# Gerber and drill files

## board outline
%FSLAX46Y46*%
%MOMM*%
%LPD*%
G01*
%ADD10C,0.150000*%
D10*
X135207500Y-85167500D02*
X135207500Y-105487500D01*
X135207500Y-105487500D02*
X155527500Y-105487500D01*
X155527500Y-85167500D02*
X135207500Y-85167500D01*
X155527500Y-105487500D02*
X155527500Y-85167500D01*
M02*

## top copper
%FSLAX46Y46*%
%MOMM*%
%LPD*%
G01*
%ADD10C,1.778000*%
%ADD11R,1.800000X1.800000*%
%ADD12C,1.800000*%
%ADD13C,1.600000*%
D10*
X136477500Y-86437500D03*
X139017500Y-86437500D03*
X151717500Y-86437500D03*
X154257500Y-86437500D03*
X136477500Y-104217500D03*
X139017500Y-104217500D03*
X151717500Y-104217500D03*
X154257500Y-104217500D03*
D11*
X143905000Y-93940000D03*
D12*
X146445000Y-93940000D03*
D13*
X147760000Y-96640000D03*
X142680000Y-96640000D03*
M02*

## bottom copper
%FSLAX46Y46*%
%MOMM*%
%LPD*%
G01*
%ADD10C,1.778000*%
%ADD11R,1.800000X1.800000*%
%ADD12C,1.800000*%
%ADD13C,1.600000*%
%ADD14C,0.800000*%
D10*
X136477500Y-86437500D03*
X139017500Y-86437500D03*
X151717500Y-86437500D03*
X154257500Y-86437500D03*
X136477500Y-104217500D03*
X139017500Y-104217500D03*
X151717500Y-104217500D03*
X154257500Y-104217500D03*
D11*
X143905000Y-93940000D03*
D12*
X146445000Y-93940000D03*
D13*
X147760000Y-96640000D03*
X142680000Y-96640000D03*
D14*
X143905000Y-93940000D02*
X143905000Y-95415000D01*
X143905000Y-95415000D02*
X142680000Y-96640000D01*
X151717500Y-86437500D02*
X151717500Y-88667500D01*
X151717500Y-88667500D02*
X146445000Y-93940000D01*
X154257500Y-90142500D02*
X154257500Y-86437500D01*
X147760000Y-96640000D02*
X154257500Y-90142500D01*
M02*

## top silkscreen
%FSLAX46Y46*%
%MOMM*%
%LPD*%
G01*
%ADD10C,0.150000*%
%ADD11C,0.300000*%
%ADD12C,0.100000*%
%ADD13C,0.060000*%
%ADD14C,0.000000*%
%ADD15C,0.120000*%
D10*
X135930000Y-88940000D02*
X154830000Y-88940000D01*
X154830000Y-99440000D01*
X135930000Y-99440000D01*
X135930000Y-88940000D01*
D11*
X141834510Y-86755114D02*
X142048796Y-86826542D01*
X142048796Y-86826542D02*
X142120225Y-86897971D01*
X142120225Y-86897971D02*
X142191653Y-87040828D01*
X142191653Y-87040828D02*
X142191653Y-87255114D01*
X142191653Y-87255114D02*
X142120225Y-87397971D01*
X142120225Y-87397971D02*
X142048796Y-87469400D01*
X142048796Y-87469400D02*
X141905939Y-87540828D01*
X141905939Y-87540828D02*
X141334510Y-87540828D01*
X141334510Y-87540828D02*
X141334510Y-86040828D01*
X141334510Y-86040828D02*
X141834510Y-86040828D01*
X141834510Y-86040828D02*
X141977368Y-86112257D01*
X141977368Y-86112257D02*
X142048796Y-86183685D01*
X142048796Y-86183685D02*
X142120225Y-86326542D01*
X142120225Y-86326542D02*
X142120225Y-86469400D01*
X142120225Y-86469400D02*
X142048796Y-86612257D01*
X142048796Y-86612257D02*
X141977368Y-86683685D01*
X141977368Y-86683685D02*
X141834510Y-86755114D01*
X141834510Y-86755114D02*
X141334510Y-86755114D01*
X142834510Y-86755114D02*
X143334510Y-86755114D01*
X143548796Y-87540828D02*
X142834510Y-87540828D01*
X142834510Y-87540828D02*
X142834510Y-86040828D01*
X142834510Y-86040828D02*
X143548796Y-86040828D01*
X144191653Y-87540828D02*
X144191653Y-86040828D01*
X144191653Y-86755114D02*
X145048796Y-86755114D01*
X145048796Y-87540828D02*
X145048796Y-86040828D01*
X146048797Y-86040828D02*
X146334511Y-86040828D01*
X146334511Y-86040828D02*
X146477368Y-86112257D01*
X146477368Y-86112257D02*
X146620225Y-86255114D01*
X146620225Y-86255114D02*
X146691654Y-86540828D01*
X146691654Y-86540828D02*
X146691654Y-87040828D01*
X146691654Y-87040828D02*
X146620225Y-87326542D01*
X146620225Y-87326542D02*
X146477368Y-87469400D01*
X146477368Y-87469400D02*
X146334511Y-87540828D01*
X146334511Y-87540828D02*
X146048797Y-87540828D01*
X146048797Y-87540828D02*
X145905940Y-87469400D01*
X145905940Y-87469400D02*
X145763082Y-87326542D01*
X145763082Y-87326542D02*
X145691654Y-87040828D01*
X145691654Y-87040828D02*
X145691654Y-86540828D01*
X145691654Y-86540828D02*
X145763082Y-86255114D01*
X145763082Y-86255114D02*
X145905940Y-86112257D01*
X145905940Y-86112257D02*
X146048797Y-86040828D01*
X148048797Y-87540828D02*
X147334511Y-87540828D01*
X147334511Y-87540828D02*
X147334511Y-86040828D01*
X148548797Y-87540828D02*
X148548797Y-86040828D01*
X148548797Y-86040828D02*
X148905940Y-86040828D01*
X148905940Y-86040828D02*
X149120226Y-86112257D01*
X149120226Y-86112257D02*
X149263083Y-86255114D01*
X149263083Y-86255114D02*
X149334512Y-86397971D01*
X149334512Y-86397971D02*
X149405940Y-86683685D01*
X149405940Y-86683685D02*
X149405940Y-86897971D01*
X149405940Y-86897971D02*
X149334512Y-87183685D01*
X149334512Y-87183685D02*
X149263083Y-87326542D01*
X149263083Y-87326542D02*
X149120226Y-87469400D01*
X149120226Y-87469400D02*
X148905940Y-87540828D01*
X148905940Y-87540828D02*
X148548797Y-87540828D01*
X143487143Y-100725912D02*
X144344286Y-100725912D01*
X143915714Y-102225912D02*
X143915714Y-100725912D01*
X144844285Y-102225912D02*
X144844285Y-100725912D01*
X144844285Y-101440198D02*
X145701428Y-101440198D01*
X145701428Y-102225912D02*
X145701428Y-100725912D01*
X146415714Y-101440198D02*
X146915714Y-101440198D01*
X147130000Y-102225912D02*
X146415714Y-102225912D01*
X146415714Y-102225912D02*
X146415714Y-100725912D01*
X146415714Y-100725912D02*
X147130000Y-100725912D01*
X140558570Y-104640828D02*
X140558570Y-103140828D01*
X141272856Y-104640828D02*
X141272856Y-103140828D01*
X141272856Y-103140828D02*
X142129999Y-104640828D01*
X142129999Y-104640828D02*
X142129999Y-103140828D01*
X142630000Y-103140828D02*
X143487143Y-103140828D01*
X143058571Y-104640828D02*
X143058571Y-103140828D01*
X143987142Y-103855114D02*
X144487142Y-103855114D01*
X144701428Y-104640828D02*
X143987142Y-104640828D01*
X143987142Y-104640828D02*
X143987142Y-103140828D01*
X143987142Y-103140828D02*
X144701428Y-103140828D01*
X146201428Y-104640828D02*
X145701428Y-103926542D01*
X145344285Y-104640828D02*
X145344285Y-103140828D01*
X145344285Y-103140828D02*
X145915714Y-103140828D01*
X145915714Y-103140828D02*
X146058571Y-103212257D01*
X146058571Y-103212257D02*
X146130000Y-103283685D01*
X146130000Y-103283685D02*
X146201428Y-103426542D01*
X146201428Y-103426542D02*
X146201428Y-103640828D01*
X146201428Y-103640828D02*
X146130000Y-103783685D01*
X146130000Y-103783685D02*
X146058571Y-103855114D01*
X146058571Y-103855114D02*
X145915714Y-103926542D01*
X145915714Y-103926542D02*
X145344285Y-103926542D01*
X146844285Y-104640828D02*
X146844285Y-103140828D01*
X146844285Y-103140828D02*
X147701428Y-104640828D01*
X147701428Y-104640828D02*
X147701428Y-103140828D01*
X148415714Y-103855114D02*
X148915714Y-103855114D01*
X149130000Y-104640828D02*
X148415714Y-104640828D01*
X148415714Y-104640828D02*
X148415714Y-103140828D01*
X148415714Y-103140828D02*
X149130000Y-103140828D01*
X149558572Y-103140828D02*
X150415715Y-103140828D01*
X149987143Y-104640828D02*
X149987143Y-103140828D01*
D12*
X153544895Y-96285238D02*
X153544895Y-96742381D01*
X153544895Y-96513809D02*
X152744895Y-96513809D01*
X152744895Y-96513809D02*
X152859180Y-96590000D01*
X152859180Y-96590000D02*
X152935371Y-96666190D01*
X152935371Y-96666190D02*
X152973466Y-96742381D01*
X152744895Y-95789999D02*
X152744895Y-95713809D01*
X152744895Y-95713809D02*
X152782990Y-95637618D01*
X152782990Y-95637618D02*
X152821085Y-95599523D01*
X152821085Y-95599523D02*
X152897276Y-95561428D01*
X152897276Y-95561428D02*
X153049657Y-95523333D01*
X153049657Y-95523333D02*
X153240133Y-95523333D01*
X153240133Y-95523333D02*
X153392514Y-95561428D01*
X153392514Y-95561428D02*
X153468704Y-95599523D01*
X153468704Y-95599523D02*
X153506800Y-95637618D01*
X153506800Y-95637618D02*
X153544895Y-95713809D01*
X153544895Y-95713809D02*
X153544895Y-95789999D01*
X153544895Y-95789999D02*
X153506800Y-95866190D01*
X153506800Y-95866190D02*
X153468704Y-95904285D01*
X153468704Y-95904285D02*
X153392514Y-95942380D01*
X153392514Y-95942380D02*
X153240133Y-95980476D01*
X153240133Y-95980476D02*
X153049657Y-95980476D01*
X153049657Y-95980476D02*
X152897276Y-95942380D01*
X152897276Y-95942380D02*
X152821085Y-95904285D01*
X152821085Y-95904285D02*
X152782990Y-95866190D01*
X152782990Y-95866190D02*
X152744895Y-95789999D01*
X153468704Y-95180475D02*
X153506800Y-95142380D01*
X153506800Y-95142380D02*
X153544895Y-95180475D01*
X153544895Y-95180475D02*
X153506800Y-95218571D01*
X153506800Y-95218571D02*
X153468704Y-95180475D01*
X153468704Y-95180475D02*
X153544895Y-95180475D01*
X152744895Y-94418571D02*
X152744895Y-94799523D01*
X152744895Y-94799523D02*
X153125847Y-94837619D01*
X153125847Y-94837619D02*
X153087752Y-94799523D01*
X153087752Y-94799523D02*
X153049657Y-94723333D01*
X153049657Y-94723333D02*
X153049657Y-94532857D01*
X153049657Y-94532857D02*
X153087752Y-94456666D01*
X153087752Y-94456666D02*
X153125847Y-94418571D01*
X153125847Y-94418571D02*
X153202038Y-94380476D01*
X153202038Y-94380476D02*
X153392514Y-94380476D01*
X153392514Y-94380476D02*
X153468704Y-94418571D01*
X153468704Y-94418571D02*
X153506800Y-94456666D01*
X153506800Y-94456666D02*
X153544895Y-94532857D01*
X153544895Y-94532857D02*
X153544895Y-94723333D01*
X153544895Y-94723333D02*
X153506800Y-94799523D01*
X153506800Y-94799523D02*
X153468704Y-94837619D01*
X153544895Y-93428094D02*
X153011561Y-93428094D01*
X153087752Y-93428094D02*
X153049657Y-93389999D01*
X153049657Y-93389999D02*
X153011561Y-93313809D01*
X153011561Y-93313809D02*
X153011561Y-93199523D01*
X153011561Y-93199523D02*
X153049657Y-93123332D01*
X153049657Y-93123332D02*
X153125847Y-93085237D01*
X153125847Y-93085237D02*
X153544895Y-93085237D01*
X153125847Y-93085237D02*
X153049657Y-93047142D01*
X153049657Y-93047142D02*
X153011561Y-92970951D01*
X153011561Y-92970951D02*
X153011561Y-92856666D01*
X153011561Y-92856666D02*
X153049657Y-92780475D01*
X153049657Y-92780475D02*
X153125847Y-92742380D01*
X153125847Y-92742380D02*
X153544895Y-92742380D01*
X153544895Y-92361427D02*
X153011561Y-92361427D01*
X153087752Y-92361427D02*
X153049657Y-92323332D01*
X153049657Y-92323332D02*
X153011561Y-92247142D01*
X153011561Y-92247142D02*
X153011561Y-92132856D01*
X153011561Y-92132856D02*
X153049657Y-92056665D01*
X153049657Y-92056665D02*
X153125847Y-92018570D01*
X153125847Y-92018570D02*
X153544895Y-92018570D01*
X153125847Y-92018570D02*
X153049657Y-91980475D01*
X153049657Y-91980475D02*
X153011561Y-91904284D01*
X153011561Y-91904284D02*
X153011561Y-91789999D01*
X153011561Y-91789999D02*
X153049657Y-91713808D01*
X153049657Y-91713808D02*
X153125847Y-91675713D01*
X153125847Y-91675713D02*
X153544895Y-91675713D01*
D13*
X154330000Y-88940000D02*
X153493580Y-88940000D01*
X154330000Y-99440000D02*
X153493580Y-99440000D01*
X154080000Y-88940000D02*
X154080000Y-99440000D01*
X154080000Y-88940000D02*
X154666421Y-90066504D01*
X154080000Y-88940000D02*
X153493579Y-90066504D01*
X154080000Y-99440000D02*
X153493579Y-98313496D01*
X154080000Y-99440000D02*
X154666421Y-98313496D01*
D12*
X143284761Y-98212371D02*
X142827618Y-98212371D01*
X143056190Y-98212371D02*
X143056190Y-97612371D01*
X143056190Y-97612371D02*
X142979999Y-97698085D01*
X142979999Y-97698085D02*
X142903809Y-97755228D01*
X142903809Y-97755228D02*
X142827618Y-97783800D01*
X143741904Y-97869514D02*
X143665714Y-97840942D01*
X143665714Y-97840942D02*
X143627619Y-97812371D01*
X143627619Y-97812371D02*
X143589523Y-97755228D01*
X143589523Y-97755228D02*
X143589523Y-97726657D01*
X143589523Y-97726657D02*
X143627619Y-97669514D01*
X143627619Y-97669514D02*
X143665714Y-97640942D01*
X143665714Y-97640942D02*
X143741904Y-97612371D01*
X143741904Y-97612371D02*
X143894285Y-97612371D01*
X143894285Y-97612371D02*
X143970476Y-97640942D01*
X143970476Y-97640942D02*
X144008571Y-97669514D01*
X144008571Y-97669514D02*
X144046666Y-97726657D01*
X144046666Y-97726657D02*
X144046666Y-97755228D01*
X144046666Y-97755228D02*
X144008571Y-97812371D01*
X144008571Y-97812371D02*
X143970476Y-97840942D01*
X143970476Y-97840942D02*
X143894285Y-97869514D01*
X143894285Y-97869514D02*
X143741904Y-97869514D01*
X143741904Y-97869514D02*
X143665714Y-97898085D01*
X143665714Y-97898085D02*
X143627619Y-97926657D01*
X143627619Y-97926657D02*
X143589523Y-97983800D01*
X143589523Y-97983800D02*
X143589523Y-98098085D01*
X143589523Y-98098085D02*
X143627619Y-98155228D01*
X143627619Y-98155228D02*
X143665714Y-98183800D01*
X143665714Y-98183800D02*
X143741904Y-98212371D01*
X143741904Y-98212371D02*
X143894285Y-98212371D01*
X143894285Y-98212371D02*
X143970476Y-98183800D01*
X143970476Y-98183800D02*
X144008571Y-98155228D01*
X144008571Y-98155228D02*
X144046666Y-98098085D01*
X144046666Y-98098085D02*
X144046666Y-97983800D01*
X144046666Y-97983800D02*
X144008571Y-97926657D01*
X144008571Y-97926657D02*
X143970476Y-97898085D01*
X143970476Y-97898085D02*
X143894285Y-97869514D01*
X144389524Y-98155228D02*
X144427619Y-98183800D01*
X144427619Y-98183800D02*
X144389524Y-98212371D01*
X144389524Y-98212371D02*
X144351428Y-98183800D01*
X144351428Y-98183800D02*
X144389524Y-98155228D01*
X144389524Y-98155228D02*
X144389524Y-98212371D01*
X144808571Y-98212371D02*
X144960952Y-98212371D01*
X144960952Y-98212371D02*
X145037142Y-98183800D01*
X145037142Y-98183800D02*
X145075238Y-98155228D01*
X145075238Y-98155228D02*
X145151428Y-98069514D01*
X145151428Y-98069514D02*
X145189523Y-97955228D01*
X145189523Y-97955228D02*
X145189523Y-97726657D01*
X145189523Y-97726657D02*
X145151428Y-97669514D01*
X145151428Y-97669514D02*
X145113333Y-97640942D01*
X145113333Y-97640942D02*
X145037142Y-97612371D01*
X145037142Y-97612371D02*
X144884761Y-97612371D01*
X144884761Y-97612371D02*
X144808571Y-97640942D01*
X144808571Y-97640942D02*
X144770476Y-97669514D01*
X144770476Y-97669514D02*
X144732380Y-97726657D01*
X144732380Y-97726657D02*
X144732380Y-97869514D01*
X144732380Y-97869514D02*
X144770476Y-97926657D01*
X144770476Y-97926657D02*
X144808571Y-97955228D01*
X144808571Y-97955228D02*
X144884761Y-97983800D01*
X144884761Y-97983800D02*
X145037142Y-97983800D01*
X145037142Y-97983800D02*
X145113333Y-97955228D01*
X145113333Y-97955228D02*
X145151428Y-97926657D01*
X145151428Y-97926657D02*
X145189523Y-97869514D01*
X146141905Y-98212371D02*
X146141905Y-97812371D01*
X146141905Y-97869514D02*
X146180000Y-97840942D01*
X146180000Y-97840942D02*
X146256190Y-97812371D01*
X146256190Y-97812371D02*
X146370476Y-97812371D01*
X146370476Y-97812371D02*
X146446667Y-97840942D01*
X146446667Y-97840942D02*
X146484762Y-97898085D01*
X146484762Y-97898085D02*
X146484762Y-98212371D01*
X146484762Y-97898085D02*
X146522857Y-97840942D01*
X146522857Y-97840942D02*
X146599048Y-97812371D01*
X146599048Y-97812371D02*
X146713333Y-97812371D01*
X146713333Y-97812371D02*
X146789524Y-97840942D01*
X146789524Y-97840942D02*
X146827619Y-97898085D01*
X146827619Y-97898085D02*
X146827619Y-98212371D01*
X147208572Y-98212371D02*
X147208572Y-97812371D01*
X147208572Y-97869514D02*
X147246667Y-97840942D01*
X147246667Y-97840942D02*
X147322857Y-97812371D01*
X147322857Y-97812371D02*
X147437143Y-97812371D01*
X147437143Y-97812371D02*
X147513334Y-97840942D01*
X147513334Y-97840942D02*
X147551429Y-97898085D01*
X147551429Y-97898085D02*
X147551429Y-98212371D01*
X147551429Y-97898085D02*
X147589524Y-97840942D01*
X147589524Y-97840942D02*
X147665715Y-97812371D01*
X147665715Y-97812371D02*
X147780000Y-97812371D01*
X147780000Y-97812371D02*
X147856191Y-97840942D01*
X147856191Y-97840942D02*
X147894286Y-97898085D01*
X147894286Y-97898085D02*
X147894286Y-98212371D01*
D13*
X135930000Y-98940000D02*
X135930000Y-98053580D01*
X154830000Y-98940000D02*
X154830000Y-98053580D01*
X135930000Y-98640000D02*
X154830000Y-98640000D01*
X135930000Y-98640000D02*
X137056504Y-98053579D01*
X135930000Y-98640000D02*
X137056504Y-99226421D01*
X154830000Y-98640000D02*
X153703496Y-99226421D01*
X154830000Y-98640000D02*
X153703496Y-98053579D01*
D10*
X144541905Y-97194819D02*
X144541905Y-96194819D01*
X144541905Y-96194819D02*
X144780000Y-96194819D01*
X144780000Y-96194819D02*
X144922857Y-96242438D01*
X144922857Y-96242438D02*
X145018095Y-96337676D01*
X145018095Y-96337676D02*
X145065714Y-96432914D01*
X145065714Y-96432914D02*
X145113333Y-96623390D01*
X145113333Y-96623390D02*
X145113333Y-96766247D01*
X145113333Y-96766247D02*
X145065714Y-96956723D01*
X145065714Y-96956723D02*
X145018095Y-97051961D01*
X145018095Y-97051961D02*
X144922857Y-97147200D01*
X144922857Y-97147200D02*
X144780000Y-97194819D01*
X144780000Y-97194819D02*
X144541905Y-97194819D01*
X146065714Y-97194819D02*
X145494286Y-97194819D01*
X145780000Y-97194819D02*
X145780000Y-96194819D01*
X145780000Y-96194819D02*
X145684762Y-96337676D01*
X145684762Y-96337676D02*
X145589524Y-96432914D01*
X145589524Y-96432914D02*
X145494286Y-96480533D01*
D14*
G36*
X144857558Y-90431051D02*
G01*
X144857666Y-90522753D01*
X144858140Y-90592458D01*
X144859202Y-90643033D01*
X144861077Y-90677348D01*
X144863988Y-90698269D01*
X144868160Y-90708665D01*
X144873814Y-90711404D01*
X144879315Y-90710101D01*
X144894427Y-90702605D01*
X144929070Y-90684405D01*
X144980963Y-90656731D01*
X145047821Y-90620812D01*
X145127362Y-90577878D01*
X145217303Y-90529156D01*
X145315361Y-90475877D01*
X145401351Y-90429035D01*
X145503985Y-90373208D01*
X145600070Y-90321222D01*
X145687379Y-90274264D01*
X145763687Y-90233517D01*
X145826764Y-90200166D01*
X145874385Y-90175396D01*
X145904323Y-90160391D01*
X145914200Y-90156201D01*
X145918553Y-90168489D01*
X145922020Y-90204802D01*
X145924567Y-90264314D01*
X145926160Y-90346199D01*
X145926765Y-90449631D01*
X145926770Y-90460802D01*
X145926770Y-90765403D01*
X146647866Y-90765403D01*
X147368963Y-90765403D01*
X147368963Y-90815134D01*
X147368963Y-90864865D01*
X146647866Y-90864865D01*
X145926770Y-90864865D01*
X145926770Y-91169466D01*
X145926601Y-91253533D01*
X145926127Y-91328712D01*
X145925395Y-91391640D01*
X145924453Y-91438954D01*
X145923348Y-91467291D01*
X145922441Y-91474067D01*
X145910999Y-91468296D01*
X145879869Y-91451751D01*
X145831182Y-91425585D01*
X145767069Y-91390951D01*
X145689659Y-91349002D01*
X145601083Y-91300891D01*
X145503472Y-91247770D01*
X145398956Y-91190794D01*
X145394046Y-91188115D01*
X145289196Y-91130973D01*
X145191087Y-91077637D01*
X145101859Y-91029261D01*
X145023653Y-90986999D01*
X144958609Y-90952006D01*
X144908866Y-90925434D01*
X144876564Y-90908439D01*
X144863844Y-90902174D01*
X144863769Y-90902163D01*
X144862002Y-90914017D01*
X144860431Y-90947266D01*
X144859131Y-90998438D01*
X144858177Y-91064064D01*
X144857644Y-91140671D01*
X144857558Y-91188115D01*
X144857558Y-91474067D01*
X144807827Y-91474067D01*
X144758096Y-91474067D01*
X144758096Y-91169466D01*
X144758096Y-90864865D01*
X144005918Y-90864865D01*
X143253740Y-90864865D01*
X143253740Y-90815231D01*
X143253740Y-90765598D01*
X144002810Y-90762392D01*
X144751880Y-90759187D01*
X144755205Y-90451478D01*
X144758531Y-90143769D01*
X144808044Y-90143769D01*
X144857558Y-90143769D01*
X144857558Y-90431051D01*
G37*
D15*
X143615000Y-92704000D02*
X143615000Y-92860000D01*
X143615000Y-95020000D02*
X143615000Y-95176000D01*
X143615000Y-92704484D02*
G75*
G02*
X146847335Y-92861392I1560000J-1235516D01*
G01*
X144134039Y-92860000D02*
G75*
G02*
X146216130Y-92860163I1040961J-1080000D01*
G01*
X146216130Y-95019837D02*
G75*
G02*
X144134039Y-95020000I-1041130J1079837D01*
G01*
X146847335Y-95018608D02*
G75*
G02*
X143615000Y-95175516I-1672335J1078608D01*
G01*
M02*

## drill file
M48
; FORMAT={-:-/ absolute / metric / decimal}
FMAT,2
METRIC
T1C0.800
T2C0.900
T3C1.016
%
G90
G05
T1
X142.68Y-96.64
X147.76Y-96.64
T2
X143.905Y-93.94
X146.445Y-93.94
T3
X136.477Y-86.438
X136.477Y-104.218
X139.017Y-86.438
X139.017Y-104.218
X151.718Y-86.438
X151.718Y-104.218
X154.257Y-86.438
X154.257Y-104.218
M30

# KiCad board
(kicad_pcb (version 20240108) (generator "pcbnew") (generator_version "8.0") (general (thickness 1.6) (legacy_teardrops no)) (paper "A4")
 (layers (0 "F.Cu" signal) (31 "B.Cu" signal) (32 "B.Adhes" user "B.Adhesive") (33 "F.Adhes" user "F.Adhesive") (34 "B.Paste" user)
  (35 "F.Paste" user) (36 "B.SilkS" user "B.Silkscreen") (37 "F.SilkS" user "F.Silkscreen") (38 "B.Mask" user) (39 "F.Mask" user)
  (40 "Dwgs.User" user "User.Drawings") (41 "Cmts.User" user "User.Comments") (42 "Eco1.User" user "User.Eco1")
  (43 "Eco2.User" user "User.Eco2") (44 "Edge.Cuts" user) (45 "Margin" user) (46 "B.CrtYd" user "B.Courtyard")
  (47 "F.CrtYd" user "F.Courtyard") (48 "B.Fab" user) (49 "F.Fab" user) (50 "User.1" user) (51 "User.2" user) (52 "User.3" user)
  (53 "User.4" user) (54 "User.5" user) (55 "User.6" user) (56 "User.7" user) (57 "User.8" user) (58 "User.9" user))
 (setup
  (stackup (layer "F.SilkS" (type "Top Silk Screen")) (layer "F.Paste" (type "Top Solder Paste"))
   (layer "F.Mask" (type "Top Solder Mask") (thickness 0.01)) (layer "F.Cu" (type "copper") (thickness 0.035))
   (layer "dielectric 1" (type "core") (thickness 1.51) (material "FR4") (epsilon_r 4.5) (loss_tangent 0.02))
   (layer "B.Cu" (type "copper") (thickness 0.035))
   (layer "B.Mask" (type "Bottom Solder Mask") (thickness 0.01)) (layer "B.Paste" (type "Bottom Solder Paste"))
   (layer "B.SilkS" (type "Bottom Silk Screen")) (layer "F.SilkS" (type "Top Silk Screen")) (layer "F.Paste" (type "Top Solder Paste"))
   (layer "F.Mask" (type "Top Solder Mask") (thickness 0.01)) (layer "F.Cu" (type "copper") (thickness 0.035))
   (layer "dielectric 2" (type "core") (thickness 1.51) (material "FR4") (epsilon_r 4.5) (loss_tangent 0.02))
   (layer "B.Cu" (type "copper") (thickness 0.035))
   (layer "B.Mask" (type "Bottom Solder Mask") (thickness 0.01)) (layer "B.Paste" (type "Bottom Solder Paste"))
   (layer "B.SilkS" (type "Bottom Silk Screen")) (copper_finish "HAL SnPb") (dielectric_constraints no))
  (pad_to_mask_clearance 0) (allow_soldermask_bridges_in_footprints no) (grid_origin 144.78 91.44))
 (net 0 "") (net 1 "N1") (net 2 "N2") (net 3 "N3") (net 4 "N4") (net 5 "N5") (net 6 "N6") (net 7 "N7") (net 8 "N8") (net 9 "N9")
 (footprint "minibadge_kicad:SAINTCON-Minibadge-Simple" (layer "F.Cu") (at 135.2075 85.1675)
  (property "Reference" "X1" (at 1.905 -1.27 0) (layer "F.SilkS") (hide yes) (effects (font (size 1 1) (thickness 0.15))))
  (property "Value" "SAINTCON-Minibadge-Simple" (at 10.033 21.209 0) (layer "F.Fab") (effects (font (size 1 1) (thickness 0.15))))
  (fp_line (start 0 0) (end 0 20.32) (stroke (width 0.15) (type solid)) (layer "Edge.Cuts"))
  (fp_line (start 0 20.32) (end 20.32 20.32) (stroke (width 0.15) (type solid)) (layer "Edge.Cuts"))
  (fp_line (start 20.32 0) (end 0 0) (stroke (width 0.15) (type solid)) (layer "Edge.Cuts"))
  (fp_line (start 20.32 20.32) (end 20.32 0) (stroke (width 0.15) (type solid)) (layer "Edge.Cuts"))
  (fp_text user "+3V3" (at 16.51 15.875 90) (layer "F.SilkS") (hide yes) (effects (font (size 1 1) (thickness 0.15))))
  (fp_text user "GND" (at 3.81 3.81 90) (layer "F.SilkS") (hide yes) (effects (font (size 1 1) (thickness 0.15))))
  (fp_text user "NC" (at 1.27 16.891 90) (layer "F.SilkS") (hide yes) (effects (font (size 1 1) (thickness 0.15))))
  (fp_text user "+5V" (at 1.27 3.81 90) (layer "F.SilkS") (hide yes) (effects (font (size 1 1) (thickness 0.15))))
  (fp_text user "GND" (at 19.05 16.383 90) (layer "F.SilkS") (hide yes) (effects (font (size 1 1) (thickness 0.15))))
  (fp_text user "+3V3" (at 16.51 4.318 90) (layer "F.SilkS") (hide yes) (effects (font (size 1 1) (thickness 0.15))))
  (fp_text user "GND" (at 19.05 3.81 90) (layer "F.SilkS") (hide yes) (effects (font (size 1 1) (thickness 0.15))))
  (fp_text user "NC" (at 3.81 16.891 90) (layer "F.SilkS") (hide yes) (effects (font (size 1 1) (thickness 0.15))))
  (pad "1" thru_hole circle (at 1.27 1.27 90) (size 1.778 1.778) (drill 1.016) (layers "*.Cu" "*.Mask") (remove_unused_layers no)
   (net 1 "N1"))
  (pad "2" thru_hole circle (at 3.81 1.27 90) (size 1.778 1.778) (drill 1.016) (layers "*.Cu" "*.Mask") (remove_unused_layers no)
   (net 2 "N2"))
  (pad "7" thru_hole circle (at 16.51 1.27 90) (size 1.778 1.778) (drill 1.016) (layers "*.Cu" "*.Mask") (remove_unused_layers no)
   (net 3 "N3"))
  (pad "8" thru_hole circle (at 19.05 1.27 90) (size 1.778 1.778) (drill 1.016) (layers "*.Cu" "*.Mask") (remove_unused_layers no)
   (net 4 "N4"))
  (pad "9" thru_hole circle (at 1.27 19.05 90) (size 1.778 1.778) (drill 1.016) (layers "*.Cu" "*.Mask") (remove_unused_layers no)
   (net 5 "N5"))
  (pad "10" thru_hole circle (at 3.81 19.05 90) (size 1.778 1.778) (drill 1.016) (layers "*.Cu" "*.Mask") (remove_unused_layers no)
   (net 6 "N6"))
  (pad "15" thru_hole circle (at 16.51 19.05 90) (size 1.778 1.778) (drill 1.016) (layers "*.Cu" "*.Mask") (remove_unused_layers no)
   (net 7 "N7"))
  (pad "16" thru_hole circle (at 19.05 19.05 90) (size 1.778 1.778) (drill 1.016) (layers "*.Cu" "*.Mask") (remove_unused_layers no)
   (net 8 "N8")))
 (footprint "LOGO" (layer "F.Cu") (at 145.33 90.84 180)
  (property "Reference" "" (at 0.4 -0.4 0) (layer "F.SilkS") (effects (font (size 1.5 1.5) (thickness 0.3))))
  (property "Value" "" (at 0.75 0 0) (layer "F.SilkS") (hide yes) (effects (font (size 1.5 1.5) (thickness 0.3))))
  (fp_poly
   (pts (xy 0.571904 -0.329466) (xy 0.571904 -0.024865) (xy 1.324082 -0.024865) (xy 2.07626 -0.024865) (xy 2.07626 0.024769)
    (xy 2.07626 0.074402) (xy 1.32719 0.077608) (xy 0.57812 0.080813) (xy 0.574795 0.388522) (xy 0.571469 0.696231) (xy 0.521956 0.696231)
    (xy 0.472442 0.696231) (xy 0.472442 0.408949) (xy 0.472334 0.317247) (xy 0.47186 0.247542) (xy 0.470798 0.196967) (xy 0.468923 0.162652)
    (xy 0.466012 0.141731) (xy 0.46184 0.131335) (xy 0.456186 0.128596) (xy 0.450685 0.129899) (xy 0.435573 0.137395) (xy 0.40093 0.155595)
    (xy 0.349037 0.183269) (xy 0.282179 0.219188) (xy 0.202638 0.262122) (xy 0.112697 0.310844) (xy 0.014639 0.364123)
    (xy -0.071351 0.410965) (xy -0.173985 0.466792) (xy -0.27007 0.518778) (xy -0.357379 0.565736) (xy -0.433687 0.606483)
    (xy -0.496764 0.639834) (xy -0.544385 0.664604) (xy -0.574323 0.679609) (xy -0.5842 0.683799) (xy -0.588553 0.671511)
    (xy -0.59202 0.635198) (xy -0.594567 0.575686) (xy -0.59616 0.493801) (xy -0.596765 0.390369) (xy -0.59677 0.379198)
    (xy -0.59677 0.074597) (xy -1.317866 0.074597) (xy -2.038963 0.074597) (xy -2.038963 0.024866) (xy -2.038963 -0.024865)
    (xy -1.317866 -0.024865) (xy -0.59677 -0.024865) (xy -0.59677 -0.329466) (xy -0.596601 -0.413533) (xy -0.596127 -0.488712)
    (xy -0.595395 -0.55164) (xy -0.594453 -0.598954) (xy -0.593348 -0.627291) (xy -0.592441 -0.634067) (xy -0.580999 -0.628296)
    (xy -0.549869 -0.611751) (xy -0.501182 -0.585585) (xy -0.437069 -0.550951) (xy -0.359659 -0.509002) (xy -0.271083 -0.460891)
    (xy -0.173472 -0.40777) (xy -0.068956 -0.350794) (xy -0.064046 -0.348115) (xy 0.040804 -0.290973) (xy 0.138913 -0.237637)
    (xy 0.228141 -0.189261) (xy 0.306347 -0.146999) (xy 0.371391 -0.112006) (xy 0.421134 -0.085434) (xy 0.453436 -0.068439)
    (xy 0.466156 -0.062174) (xy 0.466231 -0.062163) (xy 0.467998 -0.074017) (xy 0.469569 -0.107266) (xy 0.470869 -0.158438)
    (xy 0.471823 -0.224064) (xy 0.472356 -0.300671) (xy 0.472442 -0.348115) (xy 0.472442 -0.634067) (xy 0.522173 -0.634067)
    (xy 0.571904 -0.634067))
   (stroke (width 0) (type solid)) (fill solid) (layer "F.SilkS")))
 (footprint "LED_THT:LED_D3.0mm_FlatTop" (layer "F.Cu") (at 143.905 93.94)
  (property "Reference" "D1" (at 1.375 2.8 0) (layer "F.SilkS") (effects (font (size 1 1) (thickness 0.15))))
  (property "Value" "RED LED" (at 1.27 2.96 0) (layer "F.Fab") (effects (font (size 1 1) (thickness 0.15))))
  (fp_line (start -0.29 -1.236) (end -0.29 -1.08) (stroke (width 0.12) (type solid)) (layer "F.SilkS"))
  (fp_line (start -0.29 1.08) (end -0.29 1.236) (stroke (width 0.12) (type solid)) (layer "F.SilkS"))
  (fp_arc (start -0.29 -1.235516) (mid 1.366487 -1.987659) (end 2.942335 -1.078608) (stroke (width 0.12) (type solid)) (layer "F.SilkS"))
  (fp_arc (start 0.229039 -1.08) (mid 1.270117 -1.5) (end 2.31113 -1.079837) (stroke (width 0.12) (type solid)) (layer "F.SilkS"))
  (fp_arc (start 2.31113 1.079837) (mid 1.270117 1.5) (end 0.229039 1.08) (stroke (width 0.12) (type solid)) (layer "F.SilkS"))
  (fp_arc (start 2.942335 1.078608) (mid 1.366487 1.987659) (end -0.29 1.235516) (stroke (width 0.12) (type solid)) (layer "F.SilkS"))
  (pad "1" thru_hole rect (at 0 0) (size 1.8 1.8) (drill 0.9) (layers "*.Cu" "*.Mask") (remove_unused_layers no) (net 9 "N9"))
  (pad "2" thru_hole circle (at 2.54 0) (size 1.8 1.8) (drill 0.9) (layers "*.Cu" "*.Mask") (remove_unused_layers no) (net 3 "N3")))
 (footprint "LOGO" (layer "B.Cu") (at 138.23 100.49 180)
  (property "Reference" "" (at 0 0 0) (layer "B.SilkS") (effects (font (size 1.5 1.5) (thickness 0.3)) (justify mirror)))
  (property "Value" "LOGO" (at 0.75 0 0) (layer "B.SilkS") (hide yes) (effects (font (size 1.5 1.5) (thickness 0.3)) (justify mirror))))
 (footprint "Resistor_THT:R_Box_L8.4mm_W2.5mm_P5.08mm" (layer "B.Cu") (at 147.76 96.64 180)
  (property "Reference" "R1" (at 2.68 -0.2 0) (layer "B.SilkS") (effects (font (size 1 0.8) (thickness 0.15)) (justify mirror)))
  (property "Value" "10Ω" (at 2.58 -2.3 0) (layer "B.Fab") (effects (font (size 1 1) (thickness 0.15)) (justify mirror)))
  (pad "1" thru_hole circle (at 0 0 180) (size 1.6 1.6) (drill 0.8) (layers "*.Cu" "*.Mask") (remove_unused_layers no) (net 4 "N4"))
  (pad "2" thru_hole circle (at 5.08 0 180) (size 1.6 1.6) (drill 0.8) (layers "*.Cu" "*.Mask") (remove_unused_layers no) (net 9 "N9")))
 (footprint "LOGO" (layer "B.Cu") (at 145.23 101.74 180)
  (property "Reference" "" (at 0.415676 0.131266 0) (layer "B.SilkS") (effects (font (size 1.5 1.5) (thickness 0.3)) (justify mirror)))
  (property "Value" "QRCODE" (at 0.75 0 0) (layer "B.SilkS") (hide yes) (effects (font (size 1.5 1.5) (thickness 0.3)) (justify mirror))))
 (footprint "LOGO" (layer "B.Cu") (at 145.28 95.24 180)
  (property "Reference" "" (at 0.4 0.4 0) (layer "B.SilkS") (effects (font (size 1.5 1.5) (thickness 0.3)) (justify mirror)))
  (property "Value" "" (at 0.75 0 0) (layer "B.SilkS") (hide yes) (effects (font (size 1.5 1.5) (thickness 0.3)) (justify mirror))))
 (gr_rect (start 135.93 88.94) (end 154.83 99.44) (stroke (width 0.15) (type default)) (fill none) (layer "F.SilkS"))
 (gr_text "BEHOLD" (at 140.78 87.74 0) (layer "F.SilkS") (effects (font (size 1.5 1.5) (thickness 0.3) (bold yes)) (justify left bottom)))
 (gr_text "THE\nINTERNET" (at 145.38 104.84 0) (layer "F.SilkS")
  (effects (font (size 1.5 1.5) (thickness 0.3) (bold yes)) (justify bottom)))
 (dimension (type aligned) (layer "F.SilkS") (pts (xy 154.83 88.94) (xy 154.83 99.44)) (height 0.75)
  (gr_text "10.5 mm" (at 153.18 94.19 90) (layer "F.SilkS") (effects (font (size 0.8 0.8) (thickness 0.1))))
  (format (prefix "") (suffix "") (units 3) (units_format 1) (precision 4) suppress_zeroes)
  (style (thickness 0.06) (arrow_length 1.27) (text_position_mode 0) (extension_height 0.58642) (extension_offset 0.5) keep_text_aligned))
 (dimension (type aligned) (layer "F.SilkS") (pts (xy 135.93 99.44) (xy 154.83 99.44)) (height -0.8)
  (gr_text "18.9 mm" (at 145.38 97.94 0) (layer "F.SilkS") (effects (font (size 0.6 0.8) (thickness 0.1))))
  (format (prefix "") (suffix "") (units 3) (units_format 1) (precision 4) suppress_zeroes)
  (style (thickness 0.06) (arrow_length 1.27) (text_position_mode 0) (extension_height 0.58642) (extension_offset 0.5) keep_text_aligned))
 (segment (start 143.905 93.94) (end 143.905 95.415) (width 0.8) (layer "B.Cu") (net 9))
 (segment (start 143.905 95.415) (end 142.68 96.64) (width 0.8) (layer "B.Cu") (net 9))
 (segment (start 151.7175 86.4375) (end 151.7175 88.6675) (width 0.8) (layer "B.Cu") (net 3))
 (segment (start 151.7175 88.6675) (end 146.445 93.94) (width 0.8) (layer "B.Cu") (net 3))
 (segment (start 154.2575 90.1425) (end 154.2575 86.4375) (width 0.8) (layer "B.Cu") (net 4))
 (segment (start 147.76 96.64) (end 154.2575 90.1425) (width 0.8) (layer "B.Cu") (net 4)))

